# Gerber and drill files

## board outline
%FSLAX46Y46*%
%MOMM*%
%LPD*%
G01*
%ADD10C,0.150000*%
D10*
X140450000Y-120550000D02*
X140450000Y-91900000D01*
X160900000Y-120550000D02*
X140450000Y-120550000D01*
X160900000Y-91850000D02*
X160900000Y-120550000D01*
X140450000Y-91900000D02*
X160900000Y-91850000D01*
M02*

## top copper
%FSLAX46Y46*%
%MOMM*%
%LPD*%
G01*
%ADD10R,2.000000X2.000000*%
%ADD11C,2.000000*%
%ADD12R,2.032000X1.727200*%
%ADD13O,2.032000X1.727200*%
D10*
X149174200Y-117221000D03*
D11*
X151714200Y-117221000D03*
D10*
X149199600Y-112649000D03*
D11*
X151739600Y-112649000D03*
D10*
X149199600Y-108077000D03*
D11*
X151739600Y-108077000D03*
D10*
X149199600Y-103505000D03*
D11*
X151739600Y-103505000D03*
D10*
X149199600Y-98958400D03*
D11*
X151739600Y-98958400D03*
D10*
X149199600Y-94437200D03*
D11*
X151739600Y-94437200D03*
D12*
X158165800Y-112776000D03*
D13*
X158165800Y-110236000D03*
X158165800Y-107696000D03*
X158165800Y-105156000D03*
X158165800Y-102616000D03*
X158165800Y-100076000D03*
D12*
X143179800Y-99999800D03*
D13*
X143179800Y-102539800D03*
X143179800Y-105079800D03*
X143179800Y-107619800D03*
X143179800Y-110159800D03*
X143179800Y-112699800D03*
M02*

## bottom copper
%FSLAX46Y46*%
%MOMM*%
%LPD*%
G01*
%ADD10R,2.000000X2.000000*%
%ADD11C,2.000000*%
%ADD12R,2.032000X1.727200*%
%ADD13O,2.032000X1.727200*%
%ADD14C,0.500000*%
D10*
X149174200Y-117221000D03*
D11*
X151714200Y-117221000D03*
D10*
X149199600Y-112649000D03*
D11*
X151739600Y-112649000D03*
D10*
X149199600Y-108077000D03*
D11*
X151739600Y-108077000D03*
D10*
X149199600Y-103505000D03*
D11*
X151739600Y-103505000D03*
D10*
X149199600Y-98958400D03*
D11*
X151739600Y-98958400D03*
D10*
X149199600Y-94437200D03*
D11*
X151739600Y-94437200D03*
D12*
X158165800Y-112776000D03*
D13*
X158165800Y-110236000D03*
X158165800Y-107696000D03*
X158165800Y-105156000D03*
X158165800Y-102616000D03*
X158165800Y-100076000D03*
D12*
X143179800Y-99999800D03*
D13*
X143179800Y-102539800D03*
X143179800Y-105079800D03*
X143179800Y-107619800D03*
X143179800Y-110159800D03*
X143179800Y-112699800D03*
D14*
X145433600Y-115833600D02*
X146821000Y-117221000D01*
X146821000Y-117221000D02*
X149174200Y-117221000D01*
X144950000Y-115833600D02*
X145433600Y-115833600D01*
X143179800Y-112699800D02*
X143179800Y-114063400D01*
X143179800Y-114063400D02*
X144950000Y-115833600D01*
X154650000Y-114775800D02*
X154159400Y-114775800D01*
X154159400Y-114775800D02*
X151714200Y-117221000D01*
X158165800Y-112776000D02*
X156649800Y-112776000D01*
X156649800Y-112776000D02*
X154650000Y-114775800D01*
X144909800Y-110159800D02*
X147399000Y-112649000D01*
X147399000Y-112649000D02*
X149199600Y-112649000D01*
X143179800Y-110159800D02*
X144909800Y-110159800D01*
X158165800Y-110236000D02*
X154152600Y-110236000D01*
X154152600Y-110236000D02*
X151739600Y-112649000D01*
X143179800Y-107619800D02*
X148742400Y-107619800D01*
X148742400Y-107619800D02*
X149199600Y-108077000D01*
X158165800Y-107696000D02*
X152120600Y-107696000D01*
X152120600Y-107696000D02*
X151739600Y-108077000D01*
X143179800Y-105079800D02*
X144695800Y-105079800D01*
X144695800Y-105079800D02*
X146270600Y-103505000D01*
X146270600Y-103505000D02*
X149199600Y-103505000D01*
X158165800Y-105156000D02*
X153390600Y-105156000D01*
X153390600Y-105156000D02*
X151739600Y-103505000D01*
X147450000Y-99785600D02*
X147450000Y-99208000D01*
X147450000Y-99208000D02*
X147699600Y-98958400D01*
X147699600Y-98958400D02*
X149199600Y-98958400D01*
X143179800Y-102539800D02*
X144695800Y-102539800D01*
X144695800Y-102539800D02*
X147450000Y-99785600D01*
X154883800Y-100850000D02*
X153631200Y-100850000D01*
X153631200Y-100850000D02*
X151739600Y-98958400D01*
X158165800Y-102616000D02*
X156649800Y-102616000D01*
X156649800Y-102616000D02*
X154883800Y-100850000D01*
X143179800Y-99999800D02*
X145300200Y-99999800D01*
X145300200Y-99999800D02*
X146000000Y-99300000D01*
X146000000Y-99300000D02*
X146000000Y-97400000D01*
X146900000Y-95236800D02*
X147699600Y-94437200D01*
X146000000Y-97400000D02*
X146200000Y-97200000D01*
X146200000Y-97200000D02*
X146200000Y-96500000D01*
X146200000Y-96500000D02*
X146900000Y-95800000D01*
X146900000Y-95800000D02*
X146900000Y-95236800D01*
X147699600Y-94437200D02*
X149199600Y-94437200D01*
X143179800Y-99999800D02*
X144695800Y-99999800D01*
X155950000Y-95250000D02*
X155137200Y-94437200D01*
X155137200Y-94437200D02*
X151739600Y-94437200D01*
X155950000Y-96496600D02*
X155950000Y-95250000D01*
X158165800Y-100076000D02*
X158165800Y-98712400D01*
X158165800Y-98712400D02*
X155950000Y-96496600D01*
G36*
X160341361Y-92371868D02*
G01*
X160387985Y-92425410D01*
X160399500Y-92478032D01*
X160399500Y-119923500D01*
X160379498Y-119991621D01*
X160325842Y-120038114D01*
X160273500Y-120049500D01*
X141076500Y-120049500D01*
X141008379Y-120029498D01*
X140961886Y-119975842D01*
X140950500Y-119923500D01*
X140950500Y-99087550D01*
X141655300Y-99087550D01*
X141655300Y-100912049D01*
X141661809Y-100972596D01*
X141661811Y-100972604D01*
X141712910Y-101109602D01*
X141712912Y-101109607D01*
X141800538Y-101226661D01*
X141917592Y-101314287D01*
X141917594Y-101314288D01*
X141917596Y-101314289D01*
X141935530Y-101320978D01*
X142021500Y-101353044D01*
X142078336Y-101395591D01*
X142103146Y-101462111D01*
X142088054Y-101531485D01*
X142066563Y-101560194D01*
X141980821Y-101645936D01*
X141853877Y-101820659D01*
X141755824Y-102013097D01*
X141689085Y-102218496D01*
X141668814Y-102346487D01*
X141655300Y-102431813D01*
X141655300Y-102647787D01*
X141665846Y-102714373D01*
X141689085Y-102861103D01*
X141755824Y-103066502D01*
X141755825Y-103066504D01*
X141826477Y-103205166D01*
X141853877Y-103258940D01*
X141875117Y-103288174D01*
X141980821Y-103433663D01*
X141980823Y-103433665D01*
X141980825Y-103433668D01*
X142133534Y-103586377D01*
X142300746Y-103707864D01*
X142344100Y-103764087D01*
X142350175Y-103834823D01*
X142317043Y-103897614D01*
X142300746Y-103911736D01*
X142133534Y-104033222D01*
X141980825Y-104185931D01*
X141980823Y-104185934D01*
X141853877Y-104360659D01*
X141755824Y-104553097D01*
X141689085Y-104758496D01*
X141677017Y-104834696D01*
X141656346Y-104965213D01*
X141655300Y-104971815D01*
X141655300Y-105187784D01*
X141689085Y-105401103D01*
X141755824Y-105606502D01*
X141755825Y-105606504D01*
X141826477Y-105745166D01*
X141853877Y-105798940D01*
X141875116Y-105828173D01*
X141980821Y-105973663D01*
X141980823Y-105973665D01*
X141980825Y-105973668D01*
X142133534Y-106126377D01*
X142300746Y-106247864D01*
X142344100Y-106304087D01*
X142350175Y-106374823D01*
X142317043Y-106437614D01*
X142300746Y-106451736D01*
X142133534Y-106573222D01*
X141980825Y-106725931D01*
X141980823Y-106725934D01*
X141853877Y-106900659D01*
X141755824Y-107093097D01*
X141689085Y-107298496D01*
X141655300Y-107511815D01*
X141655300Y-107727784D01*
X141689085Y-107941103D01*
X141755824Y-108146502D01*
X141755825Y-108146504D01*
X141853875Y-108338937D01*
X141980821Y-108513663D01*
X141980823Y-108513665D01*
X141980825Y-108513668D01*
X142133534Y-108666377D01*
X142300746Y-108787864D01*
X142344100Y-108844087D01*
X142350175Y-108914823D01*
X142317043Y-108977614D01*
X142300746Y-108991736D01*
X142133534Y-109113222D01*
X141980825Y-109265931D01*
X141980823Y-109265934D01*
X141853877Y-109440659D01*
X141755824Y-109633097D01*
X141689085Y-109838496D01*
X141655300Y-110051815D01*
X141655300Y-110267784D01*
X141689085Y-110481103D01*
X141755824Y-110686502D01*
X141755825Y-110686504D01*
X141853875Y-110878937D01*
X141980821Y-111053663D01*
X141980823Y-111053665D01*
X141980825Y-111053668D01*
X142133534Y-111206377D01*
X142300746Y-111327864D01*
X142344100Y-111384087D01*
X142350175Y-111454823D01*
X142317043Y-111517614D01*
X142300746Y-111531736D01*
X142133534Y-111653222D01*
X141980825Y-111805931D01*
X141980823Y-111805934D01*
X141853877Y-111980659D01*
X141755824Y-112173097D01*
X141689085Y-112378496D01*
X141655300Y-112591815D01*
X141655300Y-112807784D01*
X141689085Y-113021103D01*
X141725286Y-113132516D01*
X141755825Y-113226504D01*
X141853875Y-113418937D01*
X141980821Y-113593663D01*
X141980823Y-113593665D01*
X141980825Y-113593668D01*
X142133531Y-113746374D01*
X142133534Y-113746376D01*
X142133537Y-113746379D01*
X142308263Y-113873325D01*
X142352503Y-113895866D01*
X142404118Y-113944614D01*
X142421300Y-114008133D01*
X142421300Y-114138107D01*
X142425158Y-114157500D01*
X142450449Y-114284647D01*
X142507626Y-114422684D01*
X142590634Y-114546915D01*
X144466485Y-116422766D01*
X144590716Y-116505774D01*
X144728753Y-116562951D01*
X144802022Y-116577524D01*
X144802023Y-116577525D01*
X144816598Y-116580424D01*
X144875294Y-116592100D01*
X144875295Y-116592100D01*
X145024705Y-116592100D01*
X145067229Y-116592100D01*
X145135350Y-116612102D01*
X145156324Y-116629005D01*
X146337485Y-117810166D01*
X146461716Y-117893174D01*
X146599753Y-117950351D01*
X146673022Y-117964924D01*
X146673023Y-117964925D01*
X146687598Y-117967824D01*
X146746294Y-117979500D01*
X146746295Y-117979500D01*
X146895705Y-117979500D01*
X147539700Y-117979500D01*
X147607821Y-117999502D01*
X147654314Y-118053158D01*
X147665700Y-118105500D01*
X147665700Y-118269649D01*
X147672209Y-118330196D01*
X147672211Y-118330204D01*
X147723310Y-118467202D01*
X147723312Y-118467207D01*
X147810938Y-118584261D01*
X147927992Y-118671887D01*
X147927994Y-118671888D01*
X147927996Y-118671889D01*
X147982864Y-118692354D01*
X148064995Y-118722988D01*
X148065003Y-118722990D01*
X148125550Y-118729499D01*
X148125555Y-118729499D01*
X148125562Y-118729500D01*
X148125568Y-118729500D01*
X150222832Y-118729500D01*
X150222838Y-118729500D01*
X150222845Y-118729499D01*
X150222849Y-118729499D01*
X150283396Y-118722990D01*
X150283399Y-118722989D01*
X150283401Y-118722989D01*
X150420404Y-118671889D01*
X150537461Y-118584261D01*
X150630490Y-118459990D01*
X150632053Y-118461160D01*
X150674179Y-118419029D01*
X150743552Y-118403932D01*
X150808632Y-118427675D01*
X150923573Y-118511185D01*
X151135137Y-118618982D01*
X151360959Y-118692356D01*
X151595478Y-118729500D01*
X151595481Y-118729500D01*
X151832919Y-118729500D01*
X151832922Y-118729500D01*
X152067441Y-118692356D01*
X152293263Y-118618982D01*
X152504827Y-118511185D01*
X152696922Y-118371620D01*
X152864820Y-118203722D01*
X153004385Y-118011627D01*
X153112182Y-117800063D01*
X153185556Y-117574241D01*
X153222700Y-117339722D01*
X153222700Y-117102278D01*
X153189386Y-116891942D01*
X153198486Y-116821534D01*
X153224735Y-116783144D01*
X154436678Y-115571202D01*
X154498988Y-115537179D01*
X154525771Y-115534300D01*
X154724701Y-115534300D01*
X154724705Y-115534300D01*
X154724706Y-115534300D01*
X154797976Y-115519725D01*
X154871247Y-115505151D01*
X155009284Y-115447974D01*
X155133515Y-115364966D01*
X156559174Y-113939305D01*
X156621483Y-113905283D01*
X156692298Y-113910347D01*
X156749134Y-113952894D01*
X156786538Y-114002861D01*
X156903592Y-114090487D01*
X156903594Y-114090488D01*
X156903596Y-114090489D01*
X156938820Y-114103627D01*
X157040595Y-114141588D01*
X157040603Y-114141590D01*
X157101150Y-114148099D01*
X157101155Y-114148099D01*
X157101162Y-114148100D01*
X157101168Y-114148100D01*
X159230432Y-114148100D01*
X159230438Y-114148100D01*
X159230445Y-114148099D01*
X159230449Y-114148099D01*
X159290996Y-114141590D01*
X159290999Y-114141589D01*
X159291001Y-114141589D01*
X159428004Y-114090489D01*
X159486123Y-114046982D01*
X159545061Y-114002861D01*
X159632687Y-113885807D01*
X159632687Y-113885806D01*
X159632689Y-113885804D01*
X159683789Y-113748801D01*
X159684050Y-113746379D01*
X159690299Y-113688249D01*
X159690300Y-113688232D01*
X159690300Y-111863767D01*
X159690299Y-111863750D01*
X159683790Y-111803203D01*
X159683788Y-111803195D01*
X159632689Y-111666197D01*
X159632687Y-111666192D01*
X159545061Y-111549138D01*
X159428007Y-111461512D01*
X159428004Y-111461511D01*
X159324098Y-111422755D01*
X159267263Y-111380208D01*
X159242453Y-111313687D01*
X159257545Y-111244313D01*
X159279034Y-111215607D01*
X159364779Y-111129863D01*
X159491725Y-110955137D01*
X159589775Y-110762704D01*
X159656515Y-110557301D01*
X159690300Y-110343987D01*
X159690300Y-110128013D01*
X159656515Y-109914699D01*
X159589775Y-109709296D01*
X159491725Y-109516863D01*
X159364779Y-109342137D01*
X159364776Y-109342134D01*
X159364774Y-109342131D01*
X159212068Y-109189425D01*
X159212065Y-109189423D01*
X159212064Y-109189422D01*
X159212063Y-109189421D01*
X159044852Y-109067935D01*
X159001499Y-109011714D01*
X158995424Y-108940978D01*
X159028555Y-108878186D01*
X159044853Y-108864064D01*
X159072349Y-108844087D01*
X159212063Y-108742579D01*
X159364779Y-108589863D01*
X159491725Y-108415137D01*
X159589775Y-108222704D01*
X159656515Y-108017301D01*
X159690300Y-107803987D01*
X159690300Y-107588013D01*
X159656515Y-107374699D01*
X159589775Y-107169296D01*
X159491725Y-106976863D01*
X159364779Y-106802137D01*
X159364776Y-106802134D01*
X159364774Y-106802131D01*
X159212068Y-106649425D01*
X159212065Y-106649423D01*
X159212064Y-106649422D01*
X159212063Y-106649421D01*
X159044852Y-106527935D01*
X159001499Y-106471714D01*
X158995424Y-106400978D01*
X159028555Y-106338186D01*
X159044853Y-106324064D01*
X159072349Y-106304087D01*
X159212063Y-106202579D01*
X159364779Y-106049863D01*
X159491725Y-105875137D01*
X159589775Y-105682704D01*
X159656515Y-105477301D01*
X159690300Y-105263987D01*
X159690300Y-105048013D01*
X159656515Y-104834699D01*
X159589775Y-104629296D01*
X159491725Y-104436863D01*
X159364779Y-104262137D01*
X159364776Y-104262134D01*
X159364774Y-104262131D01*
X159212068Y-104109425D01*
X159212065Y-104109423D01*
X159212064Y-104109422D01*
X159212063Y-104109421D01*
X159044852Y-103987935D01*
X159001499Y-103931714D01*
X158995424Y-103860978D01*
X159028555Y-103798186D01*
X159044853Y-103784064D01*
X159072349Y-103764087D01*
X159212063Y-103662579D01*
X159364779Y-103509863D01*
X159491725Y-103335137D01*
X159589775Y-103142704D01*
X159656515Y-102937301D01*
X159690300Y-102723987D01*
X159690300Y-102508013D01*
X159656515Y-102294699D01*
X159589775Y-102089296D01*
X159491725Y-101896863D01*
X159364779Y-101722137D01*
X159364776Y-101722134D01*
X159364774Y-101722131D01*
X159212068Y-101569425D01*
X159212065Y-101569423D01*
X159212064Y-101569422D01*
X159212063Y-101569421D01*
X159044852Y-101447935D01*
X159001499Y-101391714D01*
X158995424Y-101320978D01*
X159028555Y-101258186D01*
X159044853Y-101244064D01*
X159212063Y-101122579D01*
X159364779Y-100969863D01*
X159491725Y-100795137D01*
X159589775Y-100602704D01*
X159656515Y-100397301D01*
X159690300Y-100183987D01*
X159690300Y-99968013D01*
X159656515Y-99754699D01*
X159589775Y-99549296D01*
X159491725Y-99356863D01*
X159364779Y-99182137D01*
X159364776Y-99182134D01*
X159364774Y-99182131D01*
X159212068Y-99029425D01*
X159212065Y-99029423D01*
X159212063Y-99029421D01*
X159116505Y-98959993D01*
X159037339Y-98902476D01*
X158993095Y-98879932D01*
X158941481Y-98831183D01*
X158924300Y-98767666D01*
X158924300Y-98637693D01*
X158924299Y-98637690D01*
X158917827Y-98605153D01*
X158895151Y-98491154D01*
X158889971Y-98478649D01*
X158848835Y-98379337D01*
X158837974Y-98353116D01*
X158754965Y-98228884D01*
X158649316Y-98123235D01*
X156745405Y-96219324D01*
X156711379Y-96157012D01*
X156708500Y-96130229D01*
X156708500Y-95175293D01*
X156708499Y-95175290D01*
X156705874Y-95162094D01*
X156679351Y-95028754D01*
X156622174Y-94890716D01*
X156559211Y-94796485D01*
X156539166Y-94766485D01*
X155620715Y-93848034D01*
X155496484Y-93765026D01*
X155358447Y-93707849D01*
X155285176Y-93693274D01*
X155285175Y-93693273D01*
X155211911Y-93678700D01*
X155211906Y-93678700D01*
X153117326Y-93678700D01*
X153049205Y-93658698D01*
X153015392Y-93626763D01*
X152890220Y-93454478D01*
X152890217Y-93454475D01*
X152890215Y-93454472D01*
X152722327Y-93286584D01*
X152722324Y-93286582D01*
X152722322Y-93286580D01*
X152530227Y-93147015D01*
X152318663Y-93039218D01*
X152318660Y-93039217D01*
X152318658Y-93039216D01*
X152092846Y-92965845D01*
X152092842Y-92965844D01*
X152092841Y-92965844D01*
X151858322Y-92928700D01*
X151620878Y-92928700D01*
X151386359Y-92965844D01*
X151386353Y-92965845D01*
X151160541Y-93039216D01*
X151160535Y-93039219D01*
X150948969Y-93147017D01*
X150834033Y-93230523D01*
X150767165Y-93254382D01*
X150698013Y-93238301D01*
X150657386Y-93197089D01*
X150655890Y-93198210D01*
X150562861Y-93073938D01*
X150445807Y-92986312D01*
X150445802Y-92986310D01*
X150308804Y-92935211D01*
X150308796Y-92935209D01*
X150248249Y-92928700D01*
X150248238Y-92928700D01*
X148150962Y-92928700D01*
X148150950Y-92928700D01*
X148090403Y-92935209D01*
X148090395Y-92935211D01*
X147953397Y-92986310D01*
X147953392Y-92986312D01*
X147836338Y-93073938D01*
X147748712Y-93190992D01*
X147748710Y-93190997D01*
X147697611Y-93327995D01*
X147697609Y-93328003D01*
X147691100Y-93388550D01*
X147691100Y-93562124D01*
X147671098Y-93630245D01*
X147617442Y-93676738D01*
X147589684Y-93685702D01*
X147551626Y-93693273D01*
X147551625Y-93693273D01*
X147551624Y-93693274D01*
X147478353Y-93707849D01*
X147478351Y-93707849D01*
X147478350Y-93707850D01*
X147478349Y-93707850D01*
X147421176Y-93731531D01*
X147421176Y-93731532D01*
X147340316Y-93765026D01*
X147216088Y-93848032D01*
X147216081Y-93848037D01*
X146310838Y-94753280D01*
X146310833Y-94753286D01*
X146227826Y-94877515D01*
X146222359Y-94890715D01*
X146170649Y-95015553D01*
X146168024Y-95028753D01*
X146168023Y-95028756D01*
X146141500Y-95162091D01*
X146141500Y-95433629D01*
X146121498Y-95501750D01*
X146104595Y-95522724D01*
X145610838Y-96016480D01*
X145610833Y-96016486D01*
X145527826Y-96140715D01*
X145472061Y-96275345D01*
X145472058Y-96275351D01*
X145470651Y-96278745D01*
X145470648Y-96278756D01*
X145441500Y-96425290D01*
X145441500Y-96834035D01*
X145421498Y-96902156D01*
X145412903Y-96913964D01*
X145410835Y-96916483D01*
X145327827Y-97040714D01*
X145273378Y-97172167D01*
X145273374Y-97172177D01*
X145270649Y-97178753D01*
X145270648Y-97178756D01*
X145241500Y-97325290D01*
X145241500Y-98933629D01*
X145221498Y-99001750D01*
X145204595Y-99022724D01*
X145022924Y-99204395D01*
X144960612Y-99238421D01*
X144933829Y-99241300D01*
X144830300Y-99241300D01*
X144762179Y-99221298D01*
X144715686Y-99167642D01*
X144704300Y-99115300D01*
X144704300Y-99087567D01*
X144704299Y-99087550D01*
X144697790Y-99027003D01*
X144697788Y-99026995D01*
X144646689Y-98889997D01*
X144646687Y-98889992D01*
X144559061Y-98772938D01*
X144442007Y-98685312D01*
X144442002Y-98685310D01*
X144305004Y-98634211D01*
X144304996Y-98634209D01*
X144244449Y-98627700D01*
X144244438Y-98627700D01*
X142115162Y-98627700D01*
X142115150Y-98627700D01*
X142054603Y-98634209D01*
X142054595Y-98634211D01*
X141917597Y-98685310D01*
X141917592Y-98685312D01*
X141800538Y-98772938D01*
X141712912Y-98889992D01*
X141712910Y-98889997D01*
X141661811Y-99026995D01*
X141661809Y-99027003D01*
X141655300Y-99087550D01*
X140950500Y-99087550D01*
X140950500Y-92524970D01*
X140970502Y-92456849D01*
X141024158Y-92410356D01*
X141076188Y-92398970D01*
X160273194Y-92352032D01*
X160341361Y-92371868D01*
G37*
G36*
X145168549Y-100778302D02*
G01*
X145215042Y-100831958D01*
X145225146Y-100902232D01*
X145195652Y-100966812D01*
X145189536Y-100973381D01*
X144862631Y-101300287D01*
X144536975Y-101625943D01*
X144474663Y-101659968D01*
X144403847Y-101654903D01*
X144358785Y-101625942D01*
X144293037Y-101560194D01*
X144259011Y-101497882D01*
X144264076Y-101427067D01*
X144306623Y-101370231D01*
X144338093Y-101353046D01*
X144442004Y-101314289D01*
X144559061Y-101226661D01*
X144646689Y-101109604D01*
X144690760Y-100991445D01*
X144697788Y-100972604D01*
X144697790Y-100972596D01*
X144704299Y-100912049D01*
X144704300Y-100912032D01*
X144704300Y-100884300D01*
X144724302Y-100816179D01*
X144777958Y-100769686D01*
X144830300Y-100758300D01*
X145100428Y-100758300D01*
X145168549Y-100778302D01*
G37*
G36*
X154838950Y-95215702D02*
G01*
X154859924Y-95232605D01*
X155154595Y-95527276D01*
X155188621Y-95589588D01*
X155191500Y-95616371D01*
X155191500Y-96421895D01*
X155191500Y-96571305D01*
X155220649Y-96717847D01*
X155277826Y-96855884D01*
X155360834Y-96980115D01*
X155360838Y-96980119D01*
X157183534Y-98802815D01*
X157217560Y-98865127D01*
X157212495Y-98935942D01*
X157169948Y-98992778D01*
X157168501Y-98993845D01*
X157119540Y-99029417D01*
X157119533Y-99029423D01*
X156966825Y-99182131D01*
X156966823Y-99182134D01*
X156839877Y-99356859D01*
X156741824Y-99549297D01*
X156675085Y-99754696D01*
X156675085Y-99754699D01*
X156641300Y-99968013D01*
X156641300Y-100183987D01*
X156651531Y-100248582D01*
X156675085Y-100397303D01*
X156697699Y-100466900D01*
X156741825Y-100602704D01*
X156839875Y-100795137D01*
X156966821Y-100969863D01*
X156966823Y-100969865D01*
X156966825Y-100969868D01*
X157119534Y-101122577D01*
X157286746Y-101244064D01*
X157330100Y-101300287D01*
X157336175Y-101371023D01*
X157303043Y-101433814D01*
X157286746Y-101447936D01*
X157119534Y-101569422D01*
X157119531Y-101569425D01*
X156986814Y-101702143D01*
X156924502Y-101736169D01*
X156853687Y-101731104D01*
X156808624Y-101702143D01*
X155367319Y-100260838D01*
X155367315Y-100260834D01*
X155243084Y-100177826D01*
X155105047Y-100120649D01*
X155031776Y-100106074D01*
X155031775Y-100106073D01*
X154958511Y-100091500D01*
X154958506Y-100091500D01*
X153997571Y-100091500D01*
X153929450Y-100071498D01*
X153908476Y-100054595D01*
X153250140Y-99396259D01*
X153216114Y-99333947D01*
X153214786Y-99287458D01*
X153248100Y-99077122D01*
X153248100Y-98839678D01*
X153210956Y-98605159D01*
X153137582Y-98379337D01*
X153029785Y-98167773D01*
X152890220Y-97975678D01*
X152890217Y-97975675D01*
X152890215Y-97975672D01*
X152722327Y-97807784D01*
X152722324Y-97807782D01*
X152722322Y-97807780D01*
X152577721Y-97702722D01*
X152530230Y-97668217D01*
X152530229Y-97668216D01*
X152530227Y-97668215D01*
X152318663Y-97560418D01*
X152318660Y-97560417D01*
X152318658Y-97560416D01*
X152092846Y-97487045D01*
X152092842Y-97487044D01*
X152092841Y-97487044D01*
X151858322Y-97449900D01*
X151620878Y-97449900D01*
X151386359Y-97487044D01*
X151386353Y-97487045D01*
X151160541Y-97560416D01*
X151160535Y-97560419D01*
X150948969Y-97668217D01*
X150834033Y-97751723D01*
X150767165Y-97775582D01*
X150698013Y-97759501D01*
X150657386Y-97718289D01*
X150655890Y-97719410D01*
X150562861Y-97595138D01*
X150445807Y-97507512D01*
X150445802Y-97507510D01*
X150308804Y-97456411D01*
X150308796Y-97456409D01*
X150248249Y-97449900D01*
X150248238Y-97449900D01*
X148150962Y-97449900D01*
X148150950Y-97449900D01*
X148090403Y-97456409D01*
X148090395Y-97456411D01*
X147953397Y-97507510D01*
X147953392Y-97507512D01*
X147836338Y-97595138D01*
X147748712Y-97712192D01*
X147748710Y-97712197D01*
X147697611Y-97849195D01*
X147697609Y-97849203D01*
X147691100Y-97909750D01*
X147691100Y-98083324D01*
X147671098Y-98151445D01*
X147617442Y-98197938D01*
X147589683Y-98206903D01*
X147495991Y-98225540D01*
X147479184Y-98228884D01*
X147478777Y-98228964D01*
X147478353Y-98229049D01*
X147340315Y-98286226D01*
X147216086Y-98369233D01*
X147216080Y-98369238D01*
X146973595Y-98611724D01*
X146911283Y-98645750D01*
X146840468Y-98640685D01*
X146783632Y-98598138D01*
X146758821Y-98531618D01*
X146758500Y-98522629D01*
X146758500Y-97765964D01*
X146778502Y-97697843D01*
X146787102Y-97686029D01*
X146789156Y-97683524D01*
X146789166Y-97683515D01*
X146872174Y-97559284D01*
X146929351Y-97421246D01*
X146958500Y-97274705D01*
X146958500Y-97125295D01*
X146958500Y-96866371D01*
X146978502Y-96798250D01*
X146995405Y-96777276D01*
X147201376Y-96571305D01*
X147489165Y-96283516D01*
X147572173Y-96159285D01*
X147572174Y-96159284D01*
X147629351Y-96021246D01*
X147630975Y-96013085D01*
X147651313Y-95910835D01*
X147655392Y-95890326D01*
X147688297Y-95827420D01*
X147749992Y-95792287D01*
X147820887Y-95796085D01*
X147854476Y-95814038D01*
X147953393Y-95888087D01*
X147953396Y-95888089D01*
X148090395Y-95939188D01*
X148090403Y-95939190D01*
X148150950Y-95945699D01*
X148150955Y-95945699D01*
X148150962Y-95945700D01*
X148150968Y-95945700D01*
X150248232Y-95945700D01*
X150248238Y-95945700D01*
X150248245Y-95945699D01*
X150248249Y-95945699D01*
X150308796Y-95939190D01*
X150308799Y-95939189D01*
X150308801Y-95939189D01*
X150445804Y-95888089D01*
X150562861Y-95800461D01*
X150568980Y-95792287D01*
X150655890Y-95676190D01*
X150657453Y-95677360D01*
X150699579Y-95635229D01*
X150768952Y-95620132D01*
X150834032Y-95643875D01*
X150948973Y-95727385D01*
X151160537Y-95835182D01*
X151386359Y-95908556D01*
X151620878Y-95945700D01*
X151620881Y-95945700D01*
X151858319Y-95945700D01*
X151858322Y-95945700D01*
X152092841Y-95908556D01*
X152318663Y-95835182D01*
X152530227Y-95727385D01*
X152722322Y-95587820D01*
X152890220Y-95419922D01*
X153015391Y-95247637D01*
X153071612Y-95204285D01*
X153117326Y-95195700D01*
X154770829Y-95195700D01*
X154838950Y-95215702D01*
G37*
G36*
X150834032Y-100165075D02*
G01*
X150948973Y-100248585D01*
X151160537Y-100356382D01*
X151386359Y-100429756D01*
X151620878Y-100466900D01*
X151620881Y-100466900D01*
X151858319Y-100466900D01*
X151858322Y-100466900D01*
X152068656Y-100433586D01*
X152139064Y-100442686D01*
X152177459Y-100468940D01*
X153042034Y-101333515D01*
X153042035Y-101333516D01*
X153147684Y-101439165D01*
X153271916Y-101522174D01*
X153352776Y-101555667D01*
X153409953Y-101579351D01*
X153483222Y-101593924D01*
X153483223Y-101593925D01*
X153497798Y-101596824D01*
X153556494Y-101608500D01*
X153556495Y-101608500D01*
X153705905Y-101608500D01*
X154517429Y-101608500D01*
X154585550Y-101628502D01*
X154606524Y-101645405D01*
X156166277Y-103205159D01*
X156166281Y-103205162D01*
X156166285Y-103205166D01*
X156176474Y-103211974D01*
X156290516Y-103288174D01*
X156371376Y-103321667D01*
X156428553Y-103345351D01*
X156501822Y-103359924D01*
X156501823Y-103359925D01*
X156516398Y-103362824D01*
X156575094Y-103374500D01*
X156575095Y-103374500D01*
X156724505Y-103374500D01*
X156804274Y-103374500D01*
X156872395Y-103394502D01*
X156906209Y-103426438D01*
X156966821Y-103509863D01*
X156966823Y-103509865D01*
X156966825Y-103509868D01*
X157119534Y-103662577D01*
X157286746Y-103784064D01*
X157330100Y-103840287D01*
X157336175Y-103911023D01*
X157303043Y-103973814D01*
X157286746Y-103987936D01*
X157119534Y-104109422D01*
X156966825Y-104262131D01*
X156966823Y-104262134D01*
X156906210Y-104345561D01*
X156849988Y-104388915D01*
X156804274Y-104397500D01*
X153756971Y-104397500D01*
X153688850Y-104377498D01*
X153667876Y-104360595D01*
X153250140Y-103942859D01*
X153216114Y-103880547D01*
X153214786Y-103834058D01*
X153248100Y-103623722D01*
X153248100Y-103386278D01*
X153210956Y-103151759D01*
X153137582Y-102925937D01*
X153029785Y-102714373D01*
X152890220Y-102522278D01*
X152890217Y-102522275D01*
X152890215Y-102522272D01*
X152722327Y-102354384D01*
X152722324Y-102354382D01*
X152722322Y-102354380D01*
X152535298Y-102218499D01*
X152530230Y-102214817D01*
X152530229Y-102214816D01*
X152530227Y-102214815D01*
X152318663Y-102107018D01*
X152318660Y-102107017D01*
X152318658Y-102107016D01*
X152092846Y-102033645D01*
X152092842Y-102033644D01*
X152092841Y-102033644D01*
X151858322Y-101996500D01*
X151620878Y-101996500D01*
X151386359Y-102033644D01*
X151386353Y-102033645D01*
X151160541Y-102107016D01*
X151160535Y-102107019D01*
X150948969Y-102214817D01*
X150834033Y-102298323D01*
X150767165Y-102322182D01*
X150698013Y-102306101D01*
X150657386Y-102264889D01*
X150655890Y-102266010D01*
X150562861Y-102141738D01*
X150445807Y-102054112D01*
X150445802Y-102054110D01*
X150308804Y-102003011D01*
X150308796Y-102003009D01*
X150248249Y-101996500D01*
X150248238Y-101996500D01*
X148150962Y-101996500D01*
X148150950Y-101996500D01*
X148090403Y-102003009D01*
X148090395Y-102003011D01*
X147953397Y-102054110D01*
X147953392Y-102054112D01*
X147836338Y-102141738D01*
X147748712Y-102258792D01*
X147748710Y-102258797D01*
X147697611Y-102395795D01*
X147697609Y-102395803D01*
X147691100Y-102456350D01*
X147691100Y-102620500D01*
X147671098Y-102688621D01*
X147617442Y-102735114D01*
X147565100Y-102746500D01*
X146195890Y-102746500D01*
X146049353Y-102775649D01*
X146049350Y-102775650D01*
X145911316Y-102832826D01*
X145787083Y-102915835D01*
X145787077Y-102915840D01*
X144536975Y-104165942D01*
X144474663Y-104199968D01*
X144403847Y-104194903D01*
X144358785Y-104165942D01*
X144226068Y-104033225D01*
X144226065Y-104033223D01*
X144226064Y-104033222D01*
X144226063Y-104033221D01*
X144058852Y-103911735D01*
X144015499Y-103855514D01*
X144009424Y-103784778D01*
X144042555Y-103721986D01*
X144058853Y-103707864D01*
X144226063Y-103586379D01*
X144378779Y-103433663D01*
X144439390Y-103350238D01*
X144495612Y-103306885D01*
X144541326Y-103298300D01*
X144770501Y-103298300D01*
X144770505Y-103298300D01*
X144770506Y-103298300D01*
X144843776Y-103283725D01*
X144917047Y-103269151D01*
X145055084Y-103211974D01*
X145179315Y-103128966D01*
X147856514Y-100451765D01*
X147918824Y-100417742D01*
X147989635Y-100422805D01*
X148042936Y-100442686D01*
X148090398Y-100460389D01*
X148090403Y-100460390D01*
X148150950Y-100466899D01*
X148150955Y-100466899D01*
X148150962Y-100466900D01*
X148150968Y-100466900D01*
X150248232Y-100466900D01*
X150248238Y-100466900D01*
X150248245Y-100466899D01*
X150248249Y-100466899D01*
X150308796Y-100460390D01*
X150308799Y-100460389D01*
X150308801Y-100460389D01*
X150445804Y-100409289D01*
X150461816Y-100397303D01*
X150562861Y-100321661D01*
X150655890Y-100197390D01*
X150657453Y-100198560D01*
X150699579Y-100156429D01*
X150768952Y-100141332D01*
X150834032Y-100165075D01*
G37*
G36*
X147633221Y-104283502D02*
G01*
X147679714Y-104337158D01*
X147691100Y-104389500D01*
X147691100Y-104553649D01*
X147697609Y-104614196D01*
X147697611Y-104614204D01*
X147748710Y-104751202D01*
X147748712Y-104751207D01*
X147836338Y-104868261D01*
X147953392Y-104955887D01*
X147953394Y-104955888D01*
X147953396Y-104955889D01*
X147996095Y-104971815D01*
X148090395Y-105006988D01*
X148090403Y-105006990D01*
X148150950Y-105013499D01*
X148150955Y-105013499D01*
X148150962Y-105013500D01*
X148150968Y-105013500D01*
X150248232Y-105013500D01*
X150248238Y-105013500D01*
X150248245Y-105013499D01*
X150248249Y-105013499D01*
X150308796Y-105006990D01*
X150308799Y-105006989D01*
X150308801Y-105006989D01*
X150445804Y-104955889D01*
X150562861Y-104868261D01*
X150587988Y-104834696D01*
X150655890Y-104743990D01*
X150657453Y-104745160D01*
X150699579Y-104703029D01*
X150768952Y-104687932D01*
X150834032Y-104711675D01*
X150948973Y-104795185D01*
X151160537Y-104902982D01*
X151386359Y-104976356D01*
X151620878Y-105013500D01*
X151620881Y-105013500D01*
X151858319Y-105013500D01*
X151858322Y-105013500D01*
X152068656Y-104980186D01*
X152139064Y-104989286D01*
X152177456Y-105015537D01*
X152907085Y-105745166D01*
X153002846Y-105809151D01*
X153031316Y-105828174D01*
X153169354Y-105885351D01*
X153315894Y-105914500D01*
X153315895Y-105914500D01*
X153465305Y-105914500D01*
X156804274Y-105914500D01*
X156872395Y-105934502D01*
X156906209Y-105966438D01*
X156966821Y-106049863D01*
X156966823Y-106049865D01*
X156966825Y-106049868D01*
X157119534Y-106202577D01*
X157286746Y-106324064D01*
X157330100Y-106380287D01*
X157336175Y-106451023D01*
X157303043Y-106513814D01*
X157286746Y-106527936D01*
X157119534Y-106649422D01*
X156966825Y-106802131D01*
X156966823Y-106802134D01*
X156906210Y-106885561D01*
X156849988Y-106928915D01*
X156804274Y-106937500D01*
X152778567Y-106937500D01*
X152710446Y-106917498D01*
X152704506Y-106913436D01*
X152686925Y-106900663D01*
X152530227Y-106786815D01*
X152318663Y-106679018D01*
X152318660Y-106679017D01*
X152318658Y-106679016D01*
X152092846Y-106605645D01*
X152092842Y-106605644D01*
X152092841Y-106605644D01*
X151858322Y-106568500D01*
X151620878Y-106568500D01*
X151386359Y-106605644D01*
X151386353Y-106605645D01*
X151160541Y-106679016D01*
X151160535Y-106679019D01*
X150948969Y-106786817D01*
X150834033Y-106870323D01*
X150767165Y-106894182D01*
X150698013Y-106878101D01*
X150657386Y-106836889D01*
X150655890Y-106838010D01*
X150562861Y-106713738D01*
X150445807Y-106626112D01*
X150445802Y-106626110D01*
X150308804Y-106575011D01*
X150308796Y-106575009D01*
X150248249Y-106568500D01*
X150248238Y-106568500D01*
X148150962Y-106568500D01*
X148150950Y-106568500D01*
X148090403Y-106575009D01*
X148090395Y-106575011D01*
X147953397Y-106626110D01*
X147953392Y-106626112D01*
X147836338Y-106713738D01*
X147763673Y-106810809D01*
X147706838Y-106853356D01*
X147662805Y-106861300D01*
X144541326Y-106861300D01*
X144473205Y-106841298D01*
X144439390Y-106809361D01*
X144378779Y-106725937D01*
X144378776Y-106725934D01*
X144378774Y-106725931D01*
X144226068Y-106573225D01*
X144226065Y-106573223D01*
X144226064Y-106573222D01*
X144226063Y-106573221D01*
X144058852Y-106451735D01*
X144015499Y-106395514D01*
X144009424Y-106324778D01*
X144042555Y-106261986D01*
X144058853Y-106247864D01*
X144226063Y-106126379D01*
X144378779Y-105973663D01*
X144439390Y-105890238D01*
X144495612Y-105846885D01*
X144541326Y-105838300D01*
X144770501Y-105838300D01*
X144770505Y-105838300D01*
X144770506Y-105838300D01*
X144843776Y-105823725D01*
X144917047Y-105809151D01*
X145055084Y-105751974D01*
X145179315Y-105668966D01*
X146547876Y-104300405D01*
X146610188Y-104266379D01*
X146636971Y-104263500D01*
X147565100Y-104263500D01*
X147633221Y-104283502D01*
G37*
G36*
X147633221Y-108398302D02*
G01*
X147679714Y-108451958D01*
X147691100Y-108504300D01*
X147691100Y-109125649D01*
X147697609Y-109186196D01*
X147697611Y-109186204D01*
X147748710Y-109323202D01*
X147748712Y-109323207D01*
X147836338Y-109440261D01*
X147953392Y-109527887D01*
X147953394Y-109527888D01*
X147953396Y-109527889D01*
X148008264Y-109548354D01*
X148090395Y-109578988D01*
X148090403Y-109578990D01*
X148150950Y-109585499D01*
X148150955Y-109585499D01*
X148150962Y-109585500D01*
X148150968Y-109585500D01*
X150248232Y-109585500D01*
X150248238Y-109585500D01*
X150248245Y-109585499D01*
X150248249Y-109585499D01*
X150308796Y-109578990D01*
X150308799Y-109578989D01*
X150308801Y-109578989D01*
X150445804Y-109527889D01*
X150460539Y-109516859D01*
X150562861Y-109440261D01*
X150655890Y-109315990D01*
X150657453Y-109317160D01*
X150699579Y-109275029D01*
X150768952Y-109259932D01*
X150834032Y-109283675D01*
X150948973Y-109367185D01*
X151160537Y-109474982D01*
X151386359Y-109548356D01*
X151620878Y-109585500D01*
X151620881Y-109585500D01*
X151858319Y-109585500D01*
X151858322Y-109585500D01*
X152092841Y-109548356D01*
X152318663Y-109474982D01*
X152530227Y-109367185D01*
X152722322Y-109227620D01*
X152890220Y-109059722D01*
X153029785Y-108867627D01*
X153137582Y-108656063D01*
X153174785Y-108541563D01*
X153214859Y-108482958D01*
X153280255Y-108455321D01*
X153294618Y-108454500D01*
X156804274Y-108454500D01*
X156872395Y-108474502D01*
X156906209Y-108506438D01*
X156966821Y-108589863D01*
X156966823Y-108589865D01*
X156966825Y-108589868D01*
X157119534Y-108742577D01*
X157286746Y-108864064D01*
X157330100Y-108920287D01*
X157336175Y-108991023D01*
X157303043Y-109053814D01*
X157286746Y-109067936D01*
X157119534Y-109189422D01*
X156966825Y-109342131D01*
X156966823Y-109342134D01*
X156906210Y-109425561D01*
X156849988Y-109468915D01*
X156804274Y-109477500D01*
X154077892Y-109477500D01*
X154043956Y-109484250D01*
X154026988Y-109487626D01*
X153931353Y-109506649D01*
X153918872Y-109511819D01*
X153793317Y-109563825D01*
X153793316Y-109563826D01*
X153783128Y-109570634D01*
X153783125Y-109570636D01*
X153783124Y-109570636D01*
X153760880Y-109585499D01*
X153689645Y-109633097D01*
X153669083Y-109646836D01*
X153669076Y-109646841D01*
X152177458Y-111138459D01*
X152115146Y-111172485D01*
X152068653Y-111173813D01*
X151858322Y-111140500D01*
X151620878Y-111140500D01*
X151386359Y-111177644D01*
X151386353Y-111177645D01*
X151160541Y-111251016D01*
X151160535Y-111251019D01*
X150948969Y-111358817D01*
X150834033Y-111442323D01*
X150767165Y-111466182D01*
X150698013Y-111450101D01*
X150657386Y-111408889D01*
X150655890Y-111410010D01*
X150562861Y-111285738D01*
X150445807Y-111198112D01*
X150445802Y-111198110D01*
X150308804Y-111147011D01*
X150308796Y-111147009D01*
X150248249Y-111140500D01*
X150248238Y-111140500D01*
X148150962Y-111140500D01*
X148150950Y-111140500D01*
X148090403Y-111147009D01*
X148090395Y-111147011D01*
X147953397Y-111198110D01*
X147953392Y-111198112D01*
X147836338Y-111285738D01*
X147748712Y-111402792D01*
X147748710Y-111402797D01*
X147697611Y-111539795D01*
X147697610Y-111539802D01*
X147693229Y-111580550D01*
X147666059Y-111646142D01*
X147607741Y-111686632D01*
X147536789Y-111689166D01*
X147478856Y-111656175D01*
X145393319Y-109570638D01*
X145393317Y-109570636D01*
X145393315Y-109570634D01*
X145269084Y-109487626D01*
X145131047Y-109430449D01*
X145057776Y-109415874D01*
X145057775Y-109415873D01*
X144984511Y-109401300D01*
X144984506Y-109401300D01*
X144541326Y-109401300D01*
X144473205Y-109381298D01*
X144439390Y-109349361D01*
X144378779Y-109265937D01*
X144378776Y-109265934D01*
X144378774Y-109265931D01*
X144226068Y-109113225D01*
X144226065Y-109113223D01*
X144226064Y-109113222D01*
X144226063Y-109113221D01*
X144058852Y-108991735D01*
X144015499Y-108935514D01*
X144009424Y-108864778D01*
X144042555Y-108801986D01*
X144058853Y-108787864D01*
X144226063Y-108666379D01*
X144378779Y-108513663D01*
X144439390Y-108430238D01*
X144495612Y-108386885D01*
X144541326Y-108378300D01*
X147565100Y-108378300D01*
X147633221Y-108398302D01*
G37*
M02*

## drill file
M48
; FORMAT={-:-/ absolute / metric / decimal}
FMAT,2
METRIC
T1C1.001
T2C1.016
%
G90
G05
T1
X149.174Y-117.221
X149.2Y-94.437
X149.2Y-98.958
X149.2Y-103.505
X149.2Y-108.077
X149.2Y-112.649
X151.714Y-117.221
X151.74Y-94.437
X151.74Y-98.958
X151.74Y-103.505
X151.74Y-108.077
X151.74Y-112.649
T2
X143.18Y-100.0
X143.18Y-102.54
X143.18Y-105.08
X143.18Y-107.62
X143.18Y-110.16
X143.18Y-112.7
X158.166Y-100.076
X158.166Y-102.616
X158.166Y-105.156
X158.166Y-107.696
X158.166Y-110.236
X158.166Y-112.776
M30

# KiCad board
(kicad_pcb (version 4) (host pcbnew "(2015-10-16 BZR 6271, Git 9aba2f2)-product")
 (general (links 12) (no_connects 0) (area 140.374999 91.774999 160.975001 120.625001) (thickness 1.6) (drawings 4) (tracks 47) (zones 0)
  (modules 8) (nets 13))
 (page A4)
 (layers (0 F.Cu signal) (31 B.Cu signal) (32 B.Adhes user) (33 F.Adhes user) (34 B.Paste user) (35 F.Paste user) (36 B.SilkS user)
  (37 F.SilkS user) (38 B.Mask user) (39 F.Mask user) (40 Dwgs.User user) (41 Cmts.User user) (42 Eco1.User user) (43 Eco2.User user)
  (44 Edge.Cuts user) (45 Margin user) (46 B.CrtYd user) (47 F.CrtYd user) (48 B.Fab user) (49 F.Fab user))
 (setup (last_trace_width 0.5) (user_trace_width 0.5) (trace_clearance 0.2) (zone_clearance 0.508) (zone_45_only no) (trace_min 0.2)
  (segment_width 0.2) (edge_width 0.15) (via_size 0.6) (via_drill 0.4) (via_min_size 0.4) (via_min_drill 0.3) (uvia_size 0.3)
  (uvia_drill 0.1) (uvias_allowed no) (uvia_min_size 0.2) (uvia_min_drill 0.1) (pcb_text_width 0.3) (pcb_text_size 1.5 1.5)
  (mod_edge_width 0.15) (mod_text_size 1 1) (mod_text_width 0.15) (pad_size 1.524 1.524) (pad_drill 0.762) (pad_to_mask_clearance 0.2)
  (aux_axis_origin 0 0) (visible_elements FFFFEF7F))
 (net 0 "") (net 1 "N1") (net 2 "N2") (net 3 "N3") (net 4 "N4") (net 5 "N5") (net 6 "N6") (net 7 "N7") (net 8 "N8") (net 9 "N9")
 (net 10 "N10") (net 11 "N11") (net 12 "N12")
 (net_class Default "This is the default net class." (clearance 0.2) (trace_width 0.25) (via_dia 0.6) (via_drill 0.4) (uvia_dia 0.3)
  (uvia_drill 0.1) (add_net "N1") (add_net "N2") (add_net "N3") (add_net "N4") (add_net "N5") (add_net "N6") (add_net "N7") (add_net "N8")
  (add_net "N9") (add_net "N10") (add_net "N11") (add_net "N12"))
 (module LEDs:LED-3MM (layer F.Cu) (at 149.1742 117.221)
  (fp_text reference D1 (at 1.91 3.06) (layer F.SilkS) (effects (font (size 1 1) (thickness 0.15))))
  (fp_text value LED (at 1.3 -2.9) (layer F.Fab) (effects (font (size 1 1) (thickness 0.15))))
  (pad 1 thru_hole rect (at 0 0 90) (size 2 2) (drill 1.00076) (layers *.Cu *.Mask F.SilkS) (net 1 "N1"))
  (pad 2 thru_hole circle (at 2.54 0) (size 2 2) (drill 1.00076) (layers *.Cu *.Mask F.SilkS) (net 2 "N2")))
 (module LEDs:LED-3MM (layer F.Cu) (at 149.1996 112.649)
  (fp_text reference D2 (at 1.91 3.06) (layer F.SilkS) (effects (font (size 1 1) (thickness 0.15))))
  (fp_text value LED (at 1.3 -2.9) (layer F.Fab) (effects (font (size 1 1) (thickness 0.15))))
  (pad 1 thru_hole rect (at 0 0 90) (size 2 2) (drill 1.00076) (layers *.Cu *.Mask F.SilkS) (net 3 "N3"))
  (pad 2 thru_hole circle (at 2.54 0) (size 2 2) (drill 1.00076) (layers *.Cu *.Mask F.SilkS) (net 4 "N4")))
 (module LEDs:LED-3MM (layer F.Cu) (at 149.1996 108.077)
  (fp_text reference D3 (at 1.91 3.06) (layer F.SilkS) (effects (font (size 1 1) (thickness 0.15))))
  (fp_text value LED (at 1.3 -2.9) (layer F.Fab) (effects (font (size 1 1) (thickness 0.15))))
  (pad 1 thru_hole rect (at 0 0 90) (size 2 2) (drill 1.00076) (layers *.Cu *.Mask F.SilkS) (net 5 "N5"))
  (pad 2 thru_hole circle (at 2.54 0) (size 2 2) (drill 1.00076) (layers *.Cu *.Mask F.SilkS) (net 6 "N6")))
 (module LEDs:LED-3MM (layer F.Cu) (at 149.1996 103.505)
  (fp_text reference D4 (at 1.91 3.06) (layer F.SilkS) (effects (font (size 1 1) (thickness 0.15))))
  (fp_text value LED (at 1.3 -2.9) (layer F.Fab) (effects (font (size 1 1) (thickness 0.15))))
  (pad 1 thru_hole rect (at 0 0 90) (size 2 2) (drill 1.00076) (layers *.Cu *.Mask F.SilkS) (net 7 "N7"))
  (pad 2 thru_hole circle (at 2.54 0) (size 2 2) (drill 1.00076) (layers *.Cu *.Mask F.SilkS) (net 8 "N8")))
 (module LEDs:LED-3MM (layer F.Cu) (at 149.1996 98.9584)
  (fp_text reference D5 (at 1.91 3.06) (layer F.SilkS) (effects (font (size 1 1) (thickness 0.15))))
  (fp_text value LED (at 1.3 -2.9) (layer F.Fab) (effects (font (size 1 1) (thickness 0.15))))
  (pad 1 thru_hole rect (at 0 0 90) (size 2 2) (drill 1.00076) (layers *.Cu *.Mask F.SilkS) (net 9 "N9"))
  (pad 2 thru_hole circle (at 2.54 0) (size 2 2) (drill 1.00076) (layers *.Cu *.Mask F.SilkS) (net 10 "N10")))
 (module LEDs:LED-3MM (layer F.Cu) (at 149.1996 94.4372)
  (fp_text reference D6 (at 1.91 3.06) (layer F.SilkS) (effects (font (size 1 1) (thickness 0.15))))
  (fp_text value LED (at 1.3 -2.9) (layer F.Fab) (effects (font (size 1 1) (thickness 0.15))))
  (pad 1 thru_hole rect (at 0 0 90) (size 2 2) (drill 1.00076) (layers *.Cu *.Mask F.SilkS) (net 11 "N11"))
  (pad 2 thru_hole circle (at 2.54 0) (size 2 2) (drill 1.00076) (layers *.Cu *.Mask F.SilkS) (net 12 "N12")))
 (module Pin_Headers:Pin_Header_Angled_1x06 (layer F.Cu) (at 158.1658 112.776 180)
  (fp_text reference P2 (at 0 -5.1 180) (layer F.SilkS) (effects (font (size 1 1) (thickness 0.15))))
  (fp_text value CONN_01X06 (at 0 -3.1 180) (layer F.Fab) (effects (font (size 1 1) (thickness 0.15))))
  (pad 1 thru_hole rect (at 0 0 180) (size 2.032 1.7272) (drill 1.016) (layers *.Cu *.Mask F.SilkS) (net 2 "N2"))
  (pad 2 thru_hole oval (at 0 2.54 180) (size 2.032 1.7272) (drill 1.016) (layers *.Cu *.Mask F.SilkS) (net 4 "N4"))
  (pad 3 thru_hole oval (at 0 5.08 180) (size 2.032 1.7272) (drill 1.016) (layers *.Cu *.Mask F.SilkS) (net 6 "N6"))
  (pad 4 thru_hole oval (at 0 7.62 180) (size 2.032 1.7272) (drill 1.016) (layers *.Cu *.Mask F.SilkS) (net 8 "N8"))
  (pad 5 thru_hole oval (at 0 10.16 180) (size 2.032 1.7272) (drill 1.016) (layers *.Cu *.Mask F.SilkS) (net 10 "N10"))
  (pad 6 thru_hole oval (at 0 12.7 180) (size 2.032 1.7272) (drill 1.016) (layers *.Cu *.Mask F.SilkS) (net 12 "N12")))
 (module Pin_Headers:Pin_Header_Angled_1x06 (layer F.Cu) (at 143.1798 99.9998)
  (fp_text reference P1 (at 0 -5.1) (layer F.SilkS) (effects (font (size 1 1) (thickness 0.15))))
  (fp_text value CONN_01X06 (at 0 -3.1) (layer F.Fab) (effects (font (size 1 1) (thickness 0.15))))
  (pad 1 thru_hole rect (at 0 0) (size 2.032 1.7272) (drill 1.016) (layers *.Cu *.Mask F.SilkS) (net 11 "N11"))
  (pad 2 thru_hole oval (at 0 2.54) (size 2.032 1.7272) (drill 1.016) (layers *.Cu *.Mask F.SilkS) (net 9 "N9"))
  (pad 3 thru_hole oval (at 0 5.08) (size 2.032 1.7272) (drill 1.016) (layers *.Cu *.Mask F.SilkS) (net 7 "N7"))
  (pad 4 thru_hole oval (at 0 7.62) (size 2.032 1.7272) (drill 1.016) (layers *.Cu *.Mask F.SilkS) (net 5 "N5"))
  (pad 5 thru_hole oval (at 0 10.16) (size 2.032 1.7272) (drill 1.016) (layers *.Cu *.Mask F.SilkS) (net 3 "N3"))
  (pad 6 thru_hole oval (at 0 12.7) (size 2.032 1.7272) (drill 1.016) (layers *.Cu *.Mask F.SilkS) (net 1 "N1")))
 (gr_line (start 140.45 120.55) (end 140.45 91.9) (layer Edge.Cuts) (width 0.15))
 (gr_line (start 160.9 120.55) (end 140.45 120.55) (layer Edge.Cuts) (width 0.15))
 (gr_line (start 160.9 91.85) (end 160.9 120.55) (layer Edge.Cuts) (width 0.15))
 (gr_line (start 140.45 91.9) (end 160.9 91.85) (layer Edge.Cuts) (width 0.15))
 (segment (start 145.4336 115.8336) (end 146.821 117.221) (width 0.5) (layer B.Cu) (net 1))
 (segment (start 146.821 117.221) (end 149.1742 117.221) (width 0.5) (layer B.Cu) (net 1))
 (segment (start 144.95 115.8336) (end 145.4336 115.8336) (width 0.5) (layer B.Cu) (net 1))
 (segment (start 143.1798 112.6998) (end 143.1798 114.0634) (width 0.5) (layer B.Cu) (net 1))
 (segment (start 143.1798 114.0634) (end 144.95 115.8336) (width 0.5) (layer B.Cu) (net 1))
 (segment (start 154.65 114.7758) (end 154.1594 114.7758) (width 0.5) (layer B.Cu) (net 2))
 (segment (start 154.1594 114.7758) (end 151.7142 117.221) (width 0.5) (layer B.Cu) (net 2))
 (segment (start 158.1658 112.776) (end 156.6498 112.776) (width 0.5) (layer B.Cu) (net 2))
 (segment (start 156.6498 112.776) (end 154.65 114.7758) (width 0.5) (layer B.Cu) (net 2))
 (segment (start 144.9098 110.1598) (end 147.399 112.649) (width 0.5) (layer B.Cu) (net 3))
 (segment (start 147.399 112.649) (end 149.1996 112.649) (width 0.5) (layer B.Cu) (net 3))
 (segment (start 143.1798 110.1598) (end 144.9098 110.1598) (width 0.5) (layer B.Cu) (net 3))
 (segment (start 158.1658 110.236) (end 154.1526 110.236) (width 0.5) (layer B.Cu) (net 4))
 (segment (start 154.1526 110.236) (end 151.7396 112.649) (width 0.5) (layer B.Cu) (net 4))
 (segment (start 143.1798 107.6198) (end 148.7424 107.6198) (width 0.5) (layer B.Cu) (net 5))
 (segment (start 148.7424 107.6198) (end 149.1996 108.077) (width 0.5) (layer B.Cu) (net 5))
 (segment (start 158.1658 107.696) (end 152.1206 107.696) (width 0.5) (layer B.Cu) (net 6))
 (segment (start 152.1206 107.696) (end 151.7396 108.077) (width 0.5) (layer B.Cu) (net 6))
 (segment (start 143.1798 105.0798) (end 144.6958 105.0798) (width 0.5) (layer B.Cu) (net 7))
 (segment (start 144.6958 105.0798) (end 146.2706 103.505) (width 0.5) (layer B.Cu) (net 7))
 (segment (start 146.2706 103.505) (end 149.1996 103.505) (width 0.5) (layer B.Cu) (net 7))
 (segment (start 158.1658 105.156) (end 153.3906 105.156) (width 0.5) (layer B.Cu) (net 8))
 (segment (start 153.3906 105.156) (end 151.7396 103.505) (width 0.5) (layer B.Cu) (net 8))
 (segment (start 147.45 99.7856) (end 147.45 99.208) (width 0.5) (layer B.Cu) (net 9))
 (segment (start 147.45 99.208) (end 147.6996 98.9584) (width 0.5) (layer B.Cu) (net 9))
 (segment (start 147.6996 98.9584) (end 149.1996 98.9584) (width 0.5) (layer B.Cu) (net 9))
 (segment (start 143.1798 102.5398) (end 144.6958 102.5398) (width 0.5) (layer B.Cu) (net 9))
 (segment (start 144.6958 102.5398) (end 147.45 99.7856) (width 0.5) (layer B.Cu) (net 9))
 (segment (start 154.8838 100.85) (end 153.6312 100.85) (width 0.5) (layer B.Cu) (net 10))
 (segment (start 153.6312 100.85) (end 151.7396 98.9584) (width 0.5) (layer B.Cu) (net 10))
 (segment (start 158.1658 102.616) (end 156.6498 102.616) (width 0.5) (layer B.Cu) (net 10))
 (segment (start 156.6498 102.616) (end 154.8838 100.85) (width 0.5) (layer B.Cu) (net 10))
 (segment (start 143.1798 99.9998) (end 145.3002 99.9998) (width 0.5) (layer B.Cu) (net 11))
 (segment (start 145.3002 99.9998) (end 146 99.3) (width 0.5) (layer B.Cu) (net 11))
 (segment (start 146 99.3) (end 146 97.4) (width 0.5) (layer B.Cu) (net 11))
 (segment (start 146.9 95.2368) (end 147.6996 94.4372) (width 0.5) (layer B.Cu) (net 11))
 (segment (start 146 97.4) (end 146.2 97.2) (width 0.5) (layer B.Cu) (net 11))
 (segment (start 146.2 97.2) (end 146.2 96.5) (width 0.5) (layer B.Cu) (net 11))
 (segment (start 146.2 96.5) (end 146.9 95.8) (width 0.5) (layer B.Cu) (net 11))
 (segment (start 146.9 95.8) (end 146.9 95.2368) (width 0.5) (layer B.Cu) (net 11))
 (segment (start 147.6996 94.4372) (end 149.1996 94.4372) (width 0.5) (layer B.Cu) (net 11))
 (segment (start 143.1798 99.9998) (end 144.6958 99.9998) (width 0.5) (layer B.Cu) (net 11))
 (segment (start 155.95 95.25) (end 155.1372 94.4372) (width 0.5) (layer B.Cu) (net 12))
 (segment (start 155.1372 94.4372) (end 151.7396 94.4372) (width 0.5) (layer B.Cu) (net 12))
 (segment (start 155.95 96.4966) (end 155.95 95.25) (width 0.5) (layer B.Cu) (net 12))
 (segment (start 158.1658 100.076) (end 158.1658 98.7124) (width 0.5) (layer B.Cu) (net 12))
 (segment (start 158.1658 98.7124) (end 155.95 96.4966) (width 0.5) (layer B.Cu) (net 12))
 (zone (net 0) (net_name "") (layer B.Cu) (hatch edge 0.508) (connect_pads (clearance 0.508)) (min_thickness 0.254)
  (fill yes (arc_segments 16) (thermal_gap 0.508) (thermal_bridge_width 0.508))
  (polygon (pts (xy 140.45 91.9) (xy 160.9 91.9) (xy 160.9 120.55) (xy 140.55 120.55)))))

